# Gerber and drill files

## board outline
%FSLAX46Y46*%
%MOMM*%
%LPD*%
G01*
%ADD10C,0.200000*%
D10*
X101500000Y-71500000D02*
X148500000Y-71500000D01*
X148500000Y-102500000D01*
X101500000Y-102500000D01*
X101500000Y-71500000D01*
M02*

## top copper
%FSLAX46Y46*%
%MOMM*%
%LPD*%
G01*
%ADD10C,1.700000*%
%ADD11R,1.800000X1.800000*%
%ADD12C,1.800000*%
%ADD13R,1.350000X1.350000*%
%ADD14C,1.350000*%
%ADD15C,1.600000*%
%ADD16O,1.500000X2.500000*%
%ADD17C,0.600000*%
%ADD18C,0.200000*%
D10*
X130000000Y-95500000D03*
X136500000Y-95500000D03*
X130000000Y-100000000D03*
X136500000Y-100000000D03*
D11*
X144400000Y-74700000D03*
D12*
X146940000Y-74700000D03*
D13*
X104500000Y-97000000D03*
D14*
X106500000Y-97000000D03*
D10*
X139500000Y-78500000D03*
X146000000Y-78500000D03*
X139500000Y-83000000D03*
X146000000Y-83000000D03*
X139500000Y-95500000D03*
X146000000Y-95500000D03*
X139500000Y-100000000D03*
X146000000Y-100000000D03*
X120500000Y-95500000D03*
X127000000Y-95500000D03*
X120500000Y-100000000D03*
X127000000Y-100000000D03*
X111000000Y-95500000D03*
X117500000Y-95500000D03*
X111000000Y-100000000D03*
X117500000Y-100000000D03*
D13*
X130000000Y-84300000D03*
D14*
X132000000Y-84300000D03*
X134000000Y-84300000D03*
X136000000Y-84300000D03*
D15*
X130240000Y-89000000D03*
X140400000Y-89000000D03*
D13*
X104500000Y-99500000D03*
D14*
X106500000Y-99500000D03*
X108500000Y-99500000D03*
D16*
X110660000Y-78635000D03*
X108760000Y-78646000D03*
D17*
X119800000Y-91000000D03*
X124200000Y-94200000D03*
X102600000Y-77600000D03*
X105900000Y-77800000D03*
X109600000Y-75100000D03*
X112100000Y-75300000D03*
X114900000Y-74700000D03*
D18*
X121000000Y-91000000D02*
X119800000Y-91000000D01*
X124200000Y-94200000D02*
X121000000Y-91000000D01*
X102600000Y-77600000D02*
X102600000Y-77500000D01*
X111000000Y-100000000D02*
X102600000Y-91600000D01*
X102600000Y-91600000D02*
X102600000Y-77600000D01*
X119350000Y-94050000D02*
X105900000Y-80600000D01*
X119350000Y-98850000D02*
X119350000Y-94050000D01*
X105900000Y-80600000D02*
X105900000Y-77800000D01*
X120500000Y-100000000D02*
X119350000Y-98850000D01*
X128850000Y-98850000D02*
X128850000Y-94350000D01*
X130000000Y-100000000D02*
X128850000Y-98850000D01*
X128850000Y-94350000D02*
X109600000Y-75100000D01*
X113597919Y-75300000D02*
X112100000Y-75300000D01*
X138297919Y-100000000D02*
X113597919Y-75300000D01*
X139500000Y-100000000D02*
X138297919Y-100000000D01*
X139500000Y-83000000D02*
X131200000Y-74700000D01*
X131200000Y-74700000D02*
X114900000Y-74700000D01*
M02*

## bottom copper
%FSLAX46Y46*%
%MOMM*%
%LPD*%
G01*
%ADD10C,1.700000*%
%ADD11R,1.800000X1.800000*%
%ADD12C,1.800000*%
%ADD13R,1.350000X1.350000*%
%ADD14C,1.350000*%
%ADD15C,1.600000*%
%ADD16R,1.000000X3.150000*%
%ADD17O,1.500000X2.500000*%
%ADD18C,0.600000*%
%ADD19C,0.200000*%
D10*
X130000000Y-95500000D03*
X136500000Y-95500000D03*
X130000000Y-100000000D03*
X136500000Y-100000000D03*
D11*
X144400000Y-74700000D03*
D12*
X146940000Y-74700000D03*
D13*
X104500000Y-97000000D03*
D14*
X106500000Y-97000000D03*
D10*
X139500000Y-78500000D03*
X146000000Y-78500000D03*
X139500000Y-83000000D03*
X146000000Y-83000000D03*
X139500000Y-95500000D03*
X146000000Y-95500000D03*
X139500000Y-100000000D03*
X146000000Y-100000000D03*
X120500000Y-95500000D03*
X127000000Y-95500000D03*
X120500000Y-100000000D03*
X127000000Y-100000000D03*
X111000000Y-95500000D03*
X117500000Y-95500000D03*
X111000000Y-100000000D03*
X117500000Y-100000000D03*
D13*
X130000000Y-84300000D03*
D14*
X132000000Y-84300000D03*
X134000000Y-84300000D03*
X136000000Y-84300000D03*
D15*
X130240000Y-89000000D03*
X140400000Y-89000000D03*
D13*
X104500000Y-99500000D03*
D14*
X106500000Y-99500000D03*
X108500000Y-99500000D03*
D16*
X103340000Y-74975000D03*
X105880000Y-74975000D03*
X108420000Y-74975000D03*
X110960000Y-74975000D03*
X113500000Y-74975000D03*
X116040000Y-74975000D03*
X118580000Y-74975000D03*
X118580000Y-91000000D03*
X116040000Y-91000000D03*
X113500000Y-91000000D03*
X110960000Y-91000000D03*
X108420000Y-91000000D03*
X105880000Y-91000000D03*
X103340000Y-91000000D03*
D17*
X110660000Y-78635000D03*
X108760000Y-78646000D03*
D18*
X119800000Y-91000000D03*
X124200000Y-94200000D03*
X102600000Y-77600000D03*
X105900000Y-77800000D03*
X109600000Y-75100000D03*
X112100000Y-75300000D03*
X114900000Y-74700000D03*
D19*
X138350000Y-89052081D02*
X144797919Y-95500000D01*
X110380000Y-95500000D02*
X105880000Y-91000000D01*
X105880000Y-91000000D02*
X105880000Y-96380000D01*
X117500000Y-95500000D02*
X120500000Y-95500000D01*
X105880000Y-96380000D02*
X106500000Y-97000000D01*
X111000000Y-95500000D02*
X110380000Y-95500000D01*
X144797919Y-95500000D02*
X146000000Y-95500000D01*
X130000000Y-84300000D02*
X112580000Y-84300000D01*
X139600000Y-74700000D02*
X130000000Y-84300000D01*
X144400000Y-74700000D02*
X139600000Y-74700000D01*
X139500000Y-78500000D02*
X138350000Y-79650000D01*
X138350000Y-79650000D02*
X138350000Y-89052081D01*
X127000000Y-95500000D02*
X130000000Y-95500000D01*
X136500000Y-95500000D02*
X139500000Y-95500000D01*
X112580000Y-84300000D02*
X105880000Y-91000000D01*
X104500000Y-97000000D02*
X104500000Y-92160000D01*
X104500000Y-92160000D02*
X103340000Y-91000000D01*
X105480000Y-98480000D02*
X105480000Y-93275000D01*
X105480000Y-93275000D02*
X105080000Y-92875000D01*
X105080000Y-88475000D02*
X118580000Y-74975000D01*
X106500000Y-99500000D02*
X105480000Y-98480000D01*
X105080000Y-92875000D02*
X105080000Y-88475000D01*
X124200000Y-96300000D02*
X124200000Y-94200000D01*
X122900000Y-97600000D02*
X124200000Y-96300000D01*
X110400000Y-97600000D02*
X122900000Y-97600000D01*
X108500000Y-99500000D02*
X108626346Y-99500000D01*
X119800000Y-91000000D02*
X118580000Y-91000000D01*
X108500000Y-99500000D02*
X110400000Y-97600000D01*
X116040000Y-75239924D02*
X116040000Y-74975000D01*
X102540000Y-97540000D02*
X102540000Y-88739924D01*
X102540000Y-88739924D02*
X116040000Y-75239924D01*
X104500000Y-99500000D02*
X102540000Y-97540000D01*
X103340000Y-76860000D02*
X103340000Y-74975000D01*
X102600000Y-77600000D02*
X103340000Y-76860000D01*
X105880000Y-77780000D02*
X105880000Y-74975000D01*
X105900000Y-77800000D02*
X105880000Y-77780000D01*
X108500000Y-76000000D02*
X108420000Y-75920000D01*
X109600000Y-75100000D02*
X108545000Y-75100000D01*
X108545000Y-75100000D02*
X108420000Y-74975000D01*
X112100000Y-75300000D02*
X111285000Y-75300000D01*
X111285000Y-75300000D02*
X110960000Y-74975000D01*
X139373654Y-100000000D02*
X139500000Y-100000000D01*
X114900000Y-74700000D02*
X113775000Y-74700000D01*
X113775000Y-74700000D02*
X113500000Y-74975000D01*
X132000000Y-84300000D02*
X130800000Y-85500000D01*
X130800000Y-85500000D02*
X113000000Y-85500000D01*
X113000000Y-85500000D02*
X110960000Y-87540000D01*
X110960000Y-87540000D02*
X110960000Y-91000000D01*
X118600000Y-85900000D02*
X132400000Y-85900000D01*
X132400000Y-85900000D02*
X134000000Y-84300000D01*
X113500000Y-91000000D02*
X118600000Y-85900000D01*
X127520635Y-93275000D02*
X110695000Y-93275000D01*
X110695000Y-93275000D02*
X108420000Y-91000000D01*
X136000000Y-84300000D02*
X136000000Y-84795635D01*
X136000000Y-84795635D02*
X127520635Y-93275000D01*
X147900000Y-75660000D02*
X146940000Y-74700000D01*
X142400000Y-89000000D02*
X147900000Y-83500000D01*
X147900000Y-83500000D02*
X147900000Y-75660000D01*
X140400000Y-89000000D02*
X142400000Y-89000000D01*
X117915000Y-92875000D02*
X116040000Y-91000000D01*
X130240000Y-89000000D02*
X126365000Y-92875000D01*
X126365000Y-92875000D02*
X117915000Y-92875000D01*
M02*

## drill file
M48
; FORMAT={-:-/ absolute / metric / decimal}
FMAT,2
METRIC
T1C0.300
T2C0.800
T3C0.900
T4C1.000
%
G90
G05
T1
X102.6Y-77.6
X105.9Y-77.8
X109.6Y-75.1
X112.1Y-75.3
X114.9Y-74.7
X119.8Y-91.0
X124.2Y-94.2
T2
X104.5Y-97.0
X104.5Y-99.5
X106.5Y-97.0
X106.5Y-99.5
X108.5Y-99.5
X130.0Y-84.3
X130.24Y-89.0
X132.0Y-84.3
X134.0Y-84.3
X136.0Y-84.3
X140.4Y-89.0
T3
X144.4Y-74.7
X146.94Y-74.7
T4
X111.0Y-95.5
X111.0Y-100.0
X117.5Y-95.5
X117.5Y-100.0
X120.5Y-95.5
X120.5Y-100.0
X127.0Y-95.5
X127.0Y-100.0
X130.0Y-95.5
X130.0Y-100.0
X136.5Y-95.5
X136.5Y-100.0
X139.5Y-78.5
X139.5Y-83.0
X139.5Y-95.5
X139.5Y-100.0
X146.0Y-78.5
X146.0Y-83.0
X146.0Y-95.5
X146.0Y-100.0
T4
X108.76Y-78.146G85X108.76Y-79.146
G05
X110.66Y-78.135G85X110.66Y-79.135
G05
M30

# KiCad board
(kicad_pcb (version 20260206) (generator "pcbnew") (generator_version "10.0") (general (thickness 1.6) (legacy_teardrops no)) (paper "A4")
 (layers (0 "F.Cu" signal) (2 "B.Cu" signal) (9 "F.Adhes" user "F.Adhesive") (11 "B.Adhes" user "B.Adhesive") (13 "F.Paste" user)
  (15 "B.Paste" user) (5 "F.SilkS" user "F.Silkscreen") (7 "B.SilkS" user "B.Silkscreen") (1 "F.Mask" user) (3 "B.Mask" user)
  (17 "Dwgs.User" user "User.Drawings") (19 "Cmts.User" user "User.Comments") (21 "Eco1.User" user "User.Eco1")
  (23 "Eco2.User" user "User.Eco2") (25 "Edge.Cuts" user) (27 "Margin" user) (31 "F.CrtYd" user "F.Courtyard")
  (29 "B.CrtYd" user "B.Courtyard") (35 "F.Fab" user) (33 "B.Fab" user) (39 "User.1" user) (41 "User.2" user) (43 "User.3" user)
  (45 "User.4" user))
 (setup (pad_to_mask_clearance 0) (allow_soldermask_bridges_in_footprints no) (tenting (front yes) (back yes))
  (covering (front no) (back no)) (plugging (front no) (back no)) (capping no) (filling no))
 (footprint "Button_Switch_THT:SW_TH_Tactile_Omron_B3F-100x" (layer "F.Cu") (at 130 95.5)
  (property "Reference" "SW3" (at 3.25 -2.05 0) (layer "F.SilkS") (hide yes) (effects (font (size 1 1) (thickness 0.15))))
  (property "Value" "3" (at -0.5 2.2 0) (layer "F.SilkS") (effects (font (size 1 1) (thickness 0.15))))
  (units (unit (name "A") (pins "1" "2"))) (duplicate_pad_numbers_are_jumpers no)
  (pad "1" thru_hole circle (at 0 0) (size 1.7 1.7) (drill 1) (layers "*.Cu" "*.Mask") (remove_unused_layers no) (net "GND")
   (thermal_bridge_angle 90))
  (pad "1" thru_hole circle (at 6.5 0) (size 1.7 1.7) (drill 1) (layers "*.Cu" "*.Mask") (remove_unused_layers no) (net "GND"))
  (pad "2" thru_hole circle (at 0 4.5) (size 1.7 1.7) (drill 1) (layers "*.Cu" "*.Mask") (remove_unused_layers no) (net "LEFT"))
  (pad "2" thru_hole circle (at 6.5 4.5) (size 1.7 1.7) (drill 1) (layers "*.Cu" "*.Mask") (remove_unused_layers no) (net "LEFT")))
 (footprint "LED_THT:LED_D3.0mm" (layer "F.Cu") (at 144.4 74.7)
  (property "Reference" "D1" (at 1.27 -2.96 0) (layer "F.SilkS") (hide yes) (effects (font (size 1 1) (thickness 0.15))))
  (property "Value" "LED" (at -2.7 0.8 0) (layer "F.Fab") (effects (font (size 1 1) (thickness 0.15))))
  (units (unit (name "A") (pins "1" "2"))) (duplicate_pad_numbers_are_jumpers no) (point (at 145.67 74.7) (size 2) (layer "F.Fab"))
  (pad "1" thru_hole rect (at 0 0) (size 1.8 1.8) (drill 0.9) (layers "*.Cu" "*.Mask") (remove_unused_layers no) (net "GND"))
  (pad "2" thru_hole circle (at 2.54 0) (size 1.8 1.8) (drill 0.9) (layers "*.Cu" "*.Mask") (remove_unused_layers no) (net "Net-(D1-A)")))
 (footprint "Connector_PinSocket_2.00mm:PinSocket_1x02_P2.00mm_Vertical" (layer "F.Cu") (at 104.5 97 90)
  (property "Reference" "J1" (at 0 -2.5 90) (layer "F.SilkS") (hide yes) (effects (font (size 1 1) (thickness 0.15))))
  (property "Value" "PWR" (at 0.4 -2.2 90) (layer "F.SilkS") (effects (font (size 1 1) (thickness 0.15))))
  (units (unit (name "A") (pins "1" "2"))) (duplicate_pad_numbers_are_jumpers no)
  (pad "1" thru_hole rect (at 0 0 90) (size 1.35 1.35) (drill 0.8) (layers "*.Cu" "*.Mask") (remove_unused_layers no) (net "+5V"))
  (pad "2" thru_hole circle (at 0 2 90) (size 1.35 1.35) (drill 0.8) (layers "*.Cu" "*.Mask") (remove_unused_layers no) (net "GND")))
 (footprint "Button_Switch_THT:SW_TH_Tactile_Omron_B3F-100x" (layer "F.Cu") (at 139.5 78.5)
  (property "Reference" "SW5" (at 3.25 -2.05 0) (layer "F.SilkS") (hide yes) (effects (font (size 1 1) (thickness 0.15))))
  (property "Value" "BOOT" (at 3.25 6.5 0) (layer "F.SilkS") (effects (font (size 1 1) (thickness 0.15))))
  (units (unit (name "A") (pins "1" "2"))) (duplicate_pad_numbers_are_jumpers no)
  (pad "1" thru_hole circle (at 0 0) (size 1.7 1.7) (drill 1) (layers "*.Cu" "*.Mask") (remove_unused_layers no) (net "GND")
   (thermal_bridge_angle 90))
  (pad "1" thru_hole circle (at 6.5 0) (size 1.7 1.7) (drill 1) (layers "*.Cu" "*.Mask") (remove_unused_layers no) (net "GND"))
  (pad "2" thru_hole circle (at 0 4.5) (size 1.7 1.7) (drill 1) (layers "*.Cu" "*.Mask") (remove_unused_layers no) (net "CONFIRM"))
  (pad "2" thru_hole circle (at 6.5 4.5) (size 1.7 1.7) (drill 1) (layers "*.Cu" "*.Mask") (remove_unused_layers no) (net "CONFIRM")))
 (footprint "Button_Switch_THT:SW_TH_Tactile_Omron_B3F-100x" (layer "F.Cu") (at 139.5 95.5)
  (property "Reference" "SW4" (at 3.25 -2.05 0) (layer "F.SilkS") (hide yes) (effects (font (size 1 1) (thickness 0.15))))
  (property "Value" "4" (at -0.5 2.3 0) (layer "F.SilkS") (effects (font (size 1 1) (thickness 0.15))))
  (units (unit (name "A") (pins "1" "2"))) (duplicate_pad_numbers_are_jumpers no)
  (pad "1" thru_hole circle (at 0 0) (size 1.7 1.7) (drill 1) (layers "*.Cu" "*.Mask") (remove_unused_layers no) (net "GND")
   (thermal_bridge_angle 90))
  (pad "1" thru_hole circle (at 6.5 0) (size 1.7 1.7) (drill 1) (layers "*.Cu" "*.Mask") (remove_unused_layers no) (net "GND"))
  (pad "2" thru_hole circle (at 0 4.5) (size 1.7 1.7) (drill 1) (layers "*.Cu" "*.Mask") (remove_unused_layers no) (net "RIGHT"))
  (pad "2" thru_hole circle (at 6.5 4.5) (size 1.7 1.7) (drill 1) (layers "*.Cu" "*.Mask") (remove_unused_layers no) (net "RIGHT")))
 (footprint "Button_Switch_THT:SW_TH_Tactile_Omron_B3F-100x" (layer "F.Cu") (at 120.5 95.5)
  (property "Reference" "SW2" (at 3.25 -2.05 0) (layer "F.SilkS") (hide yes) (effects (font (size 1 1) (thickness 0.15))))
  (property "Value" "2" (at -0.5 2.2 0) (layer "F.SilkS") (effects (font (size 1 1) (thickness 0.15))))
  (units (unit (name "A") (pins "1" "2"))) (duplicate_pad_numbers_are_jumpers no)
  (pad "1" thru_hole circle (at 0 0) (size 1.7 1.7) (drill 1) (layers "*.Cu" "*.Mask") (remove_unused_layers no) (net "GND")
   (thermal_bridge_angle 90))
  (pad "1" thru_hole circle (at 6.5 0) (size 1.7 1.7) (drill 1) (layers "*.Cu" "*.Mask") (remove_unused_layers no) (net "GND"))
  (pad "2" thru_hole circle (at 0 4.5) (size 1.7 1.7) (drill 1) (layers "*.Cu" "*.Mask") (remove_unused_layers no) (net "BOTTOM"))
  (pad "2" thru_hole circle (at 6.5 4.5) (size 1.7 1.7) (drill 1) (layers "*.Cu" "*.Mask") (remove_unused_layers no) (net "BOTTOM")))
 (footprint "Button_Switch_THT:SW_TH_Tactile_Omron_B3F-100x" (layer "F.Cu") (at 111 95.5)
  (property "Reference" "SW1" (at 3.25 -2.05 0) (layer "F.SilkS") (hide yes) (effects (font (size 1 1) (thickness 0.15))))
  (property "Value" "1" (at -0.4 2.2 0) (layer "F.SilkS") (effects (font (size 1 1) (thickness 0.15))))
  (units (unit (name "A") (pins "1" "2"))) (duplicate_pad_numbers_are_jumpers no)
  (pad "1" thru_hole circle (at 0 0) (size 1.7 1.7) (drill 1) (layers "*.Cu" "*.Mask") (remove_unused_layers no) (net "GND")
   (thermal_bridge_angle 90))
  (pad "1" thru_hole circle (at 6.5 0) (size 1.7 1.7) (drill 1) (layers "*.Cu" "*.Mask") (remove_unused_layers no) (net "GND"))
  (pad "2" thru_hole circle (at 0 4.5) (size 1.7 1.7) (drill 1) (layers "*.Cu" "*.Mask") (remove_unused_layers no) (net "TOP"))
  (pad "2" thru_hole circle (at 6.5 4.5) (size 1.7 1.7) (drill 1) (layers "*.Cu" "*.Mask") (remove_unused_layers no) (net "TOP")))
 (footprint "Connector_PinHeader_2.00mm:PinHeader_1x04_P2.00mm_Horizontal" (layer "F.Cu") (at 130 84.3 90)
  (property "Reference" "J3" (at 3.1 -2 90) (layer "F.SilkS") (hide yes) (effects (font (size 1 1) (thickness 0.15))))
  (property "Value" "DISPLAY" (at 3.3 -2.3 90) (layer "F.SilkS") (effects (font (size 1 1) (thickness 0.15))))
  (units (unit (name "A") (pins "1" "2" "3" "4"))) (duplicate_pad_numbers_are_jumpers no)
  (pad "1" thru_hole rect (at 0 0 90) (size 1.35 1.35) (drill 0.8) (layers "*.Cu" "*.Mask") (remove_unused_layers no) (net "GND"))
  (pad "2" thru_hole circle (at 0 2 90) (size 1.35 1.35) (drill 0.8) (layers "*.Cu" "*.Mask") (remove_unused_layers no) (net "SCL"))
  (pad "3" thru_hole circle (at 0 4 90) (size 1.35 1.35) (drill 0.8) (layers "*.Cu" "*.Mask") (remove_unused_layers no) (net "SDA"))
  (pad "4" thru_hole circle (at 0 6 90) (size 1.35 1.35) (drill 0.8) (layers "*.Cu" "*.Mask") (remove_unused_layers no) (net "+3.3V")))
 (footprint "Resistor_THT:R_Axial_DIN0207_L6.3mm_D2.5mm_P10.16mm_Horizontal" (layer "F.Cu") (at 130.24 89)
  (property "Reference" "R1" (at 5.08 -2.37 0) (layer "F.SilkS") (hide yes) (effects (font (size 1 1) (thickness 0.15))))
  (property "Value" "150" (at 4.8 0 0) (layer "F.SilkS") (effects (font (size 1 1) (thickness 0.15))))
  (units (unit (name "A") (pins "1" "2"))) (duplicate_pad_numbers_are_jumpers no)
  (pad "1" thru_hole circle (at 0 0) (size 1.6 1.6) (drill 0.8) (layers "*.Cu" "*.Mask") (remove_unused_layers no) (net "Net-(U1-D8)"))
  (pad "2" thru_hole circle (at 10.16 0) (size 1.6 1.6) (drill 0.8) (layers "*.Cu" "*.Mask") (remove_unused_layers no) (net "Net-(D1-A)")))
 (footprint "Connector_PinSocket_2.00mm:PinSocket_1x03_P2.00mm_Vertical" (layer "F.Cu") (at 104.5 99.5 90)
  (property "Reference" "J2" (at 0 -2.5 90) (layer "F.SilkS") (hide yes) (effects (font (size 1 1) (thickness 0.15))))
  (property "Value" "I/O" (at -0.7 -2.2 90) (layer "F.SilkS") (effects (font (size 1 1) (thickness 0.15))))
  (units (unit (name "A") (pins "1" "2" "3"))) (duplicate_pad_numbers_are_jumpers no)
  (pad "1" thru_hole rect (at 0 0 90) (size 1.35 1.35) (drill 0.8) (layers "*.Cu" "*.Mask") (remove_unused_layers no) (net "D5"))
  (pad "2" thru_hole circle (at 0 2 90) (size 1.35 1.35) (drill 0.8) (layers "*.Cu" "*.Mask") (remove_unused_layers no) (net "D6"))
  (pad "3" thru_hole circle (at 0 4 90) (size 1.35 1.35) (drill 0.8) (layers "*.Cu" "*.Mask") (remove_unused_layers no) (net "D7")))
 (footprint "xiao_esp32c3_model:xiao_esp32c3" (layer "B.Cu") (at 112.76 83.575 -90)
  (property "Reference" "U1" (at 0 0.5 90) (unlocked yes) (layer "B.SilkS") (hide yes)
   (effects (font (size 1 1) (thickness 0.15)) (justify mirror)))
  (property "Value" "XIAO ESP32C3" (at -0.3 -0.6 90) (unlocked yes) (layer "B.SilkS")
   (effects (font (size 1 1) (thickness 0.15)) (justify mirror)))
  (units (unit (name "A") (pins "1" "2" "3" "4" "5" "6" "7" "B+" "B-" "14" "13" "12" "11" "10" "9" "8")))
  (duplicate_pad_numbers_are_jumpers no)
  (pad "1" smd rect (at -8.6 9.42 270) (size 3.15 1) (layers "B.Cu" "B.Mask" "B.Paste") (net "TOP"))
  (pad "2" smd rect (at -8.6 6.88 270) (size 3.15 1) (layers "B.Cu" "B.Mask" "B.Paste") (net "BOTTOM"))
  (pad "3" smd rect (at -8.6 4.34 270) (size 3.15 1) (layers "B.Cu" "B.Mask" "B.Paste") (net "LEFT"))
  (pad "4" smd rect (at -8.6 1.8 270) (size 3.15 1) (layers "B.Cu" "B.Mask" "B.Paste") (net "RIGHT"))
  (pad "5" smd rect (at -8.6 -0.74 270) (size 3.15 1) (layers "B.Cu" "B.Mask" "B.Paste") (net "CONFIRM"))
  (pad "6" smd rect (at -8.6 -3.28 270) (size 3.15 1) (layers "B.Cu" "B.Mask" "B.Paste") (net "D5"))
  (pad "7" smd rect (at -8.6 -5.82 270) (size 3.15 1) (layers "B.Cu" "B.Mask" "B.Paste") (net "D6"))
  (pad "8" smd rect (at 7.425 -5.82 270) (size 3.15 1) (layers "B.Cu" "B.Mask" "B.Paste") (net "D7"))
  (pad "9" smd rect (at 7.425 -3.28 270) (size 3.15 1) (layers "B.Cu" "B.Mask" "B.Paste") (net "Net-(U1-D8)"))
  (pad "10" smd rect (at 7.425 -0.74 270) (size 3.15 1) (layers "B.Cu" "B.Mask" "B.Paste") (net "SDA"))
  (pad "11" smd rect (at 7.425 1.8 270) (size 3.15 1) (layers "B.Cu" "B.Mask" "B.Paste") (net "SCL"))
  (pad "12" smd rect (at 7.425 4.34 270) (size 3.15 1) (layers "B.Cu" "B.Mask" "B.Paste") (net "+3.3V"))
  (pad "13" smd rect (at 7.425 6.88 270) (size 3.15 1) (layers "B.Cu" "B.Mask" "B.Paste") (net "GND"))
  (pad "14" smd rect (at 7.425 9.42 270) (size 3.15 1) (layers "B.Cu" "B.Mask" "B.Paste") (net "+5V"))
  (pad "B+" thru_hole oval (at -4.94 2.1 270) (size 2.5 1.5) (drill oval 2 1) (layers "*.Cu" "*.Mask") (remove_unused_layers no)
   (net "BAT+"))
  (pad "B-" thru_hole oval (at -4.929 4 270) (size 2.5 1.5) (drill oval 2 1) (layers "*.Cu" "*.Mask") (remove_unused_layers no) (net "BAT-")))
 (gr_rect (start 101.5 71.5) (end 148.5 102.5) (stroke (width 0.2) (type default)) (fill no) (layer "Edge.Cuts"))
 (segment (start 138.35 89.052081) (end 144.797919 95.5) (width 0.2) (layer "B.Cu") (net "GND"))
 (segment (start 110.38 95.5) (end 105.88 91) (width 0.2) (layer "B.Cu") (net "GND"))
 (segment (start 105.88 91) (end 105.88 96.38) (width 0.2) (layer "B.Cu") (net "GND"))
 (segment (start 117.5 95.5) (end 120.5 95.5) (width 0.2) (layer "B.Cu") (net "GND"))
 (segment (start 105.88 96.38) (end 106.5 97) (width 0.2) (layer "B.Cu") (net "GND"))
 (segment (start 111 95.5) (end 110.38 95.5) (width 0.2) (layer "B.Cu") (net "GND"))
 (segment (start 144.797919 95.5) (end 146 95.5) (width 0.2) (layer "B.Cu") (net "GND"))
 (segment (start 130 84.3) (end 112.58 84.3) (width 0.2) (layer "B.Cu") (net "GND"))
 (segment (start 139.6 74.7) (end 130 84.3) (width 0.2) (layer "B.Cu") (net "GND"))
 (segment (start 144.4 74.7) (end 139.6 74.7) (width 0.2) (layer "B.Cu") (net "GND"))
 (segment (start 139.5 78.5) (end 138.35 79.65) (width 0.2) (layer "B.Cu") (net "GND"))
 (segment (start 138.35 79.65) (end 138.35 89.052081) (width 0.2) (layer "B.Cu") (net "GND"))
 (segment (start 127 95.5) (end 130 95.5) (width 0.2) (layer "B.Cu") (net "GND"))
 (segment (start 136.5 95.5) (end 139.5 95.5) (width 0.2) (layer "B.Cu") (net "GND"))
 (segment (start 112.58 84.3) (end 105.88 91) (width 0.2) (layer "B.Cu") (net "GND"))
 (segment (start 104.5 97) (end 104.5 92.16) (width 0.2) (layer "B.Cu") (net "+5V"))
 (segment (start 104.5 92.16) (end 103.34 91) (width 0.2) (layer "B.Cu") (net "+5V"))
 (segment (start 105.48 98.48) (end 105.48 93.275) (width 0.2) (layer "B.Cu") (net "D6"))
 (segment (start 105.48 93.275) (end 105.08 92.875) (width 0.2) (layer "B.Cu") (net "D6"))
 (segment (start 105.08 88.475) (end 118.58 74.975) (width 0.2) (layer "B.Cu") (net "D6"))
 (segment (start 106.5 99.5) (end 105.48 98.48) (width 0.2) (layer "B.Cu") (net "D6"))
 (segment (start 105.08 92.875) (end 105.08 88.475) (width 0.2) (layer "B.Cu") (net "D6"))
 (segment (start 121 91) (end 119.8 91) (width 0.2) (layer "F.Cu") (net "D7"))
 (segment (start 124.2 94.2) (end 121 91) (width 0.2) (layer "F.Cu") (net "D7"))
 (via (at 119.8 91) (size 0.6) (drill 0.3) (layers "F.Cu" "B.Cu") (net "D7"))
 (via (at 124.2 94.2) (size 0.6) (drill 0.3) (layers "F.Cu" "B.Cu") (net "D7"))
 (segment (start 124.2 96.3) (end 124.2 94.2) (width 0.2) (layer "B.Cu") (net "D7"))
 (segment (start 122.9 97.6) (end 124.2 96.3) (width 0.2) (layer "B.Cu") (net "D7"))
 (segment (start 110.4 97.6) (end 122.9 97.6) (width 0.2) (layer "B.Cu") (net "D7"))
 (segment (start 108.5 99.5) (end 108.626346 99.5) (width 0.2) (layer "B.Cu") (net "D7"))
 (segment (start 119.8 91) (end 118.58 91) (width 0.2) (layer "B.Cu") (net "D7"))
 (segment (start 108.5 99.5) (end 110.4 97.6) (width 0.2) (layer "B.Cu") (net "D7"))
 (segment (start 116.04 75.239924) (end 116.04 74.975) (width 0.2) (layer "B.Cu") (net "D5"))
 (segment (start 102.54 97.54) (end 102.54 88.739924) (width 0.2) (layer "B.Cu") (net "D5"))
 (segment (start 102.54 88.739924) (end 116.04 75.239924) (width 0.2) (layer "B.Cu") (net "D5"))
 (segment (start 104.5 99.5) (end 102.54 97.54) (width 0.2) (layer "B.Cu") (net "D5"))
 (segment (start 102.6 77.6) (end 102.6 77.5) (width 0.2) (layer "F.Cu") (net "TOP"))
 (segment (start 111 100) (end 102.6 91.6) (width 0.2) (layer "F.Cu") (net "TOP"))
 (segment (start 102.6 91.6) (end 102.6 77.6) (width 0.2) (layer "F.Cu") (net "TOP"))
 (via (at 102.6 77.6) (size 0.6) (drill 0.3) (layers "F.Cu" "B.Cu") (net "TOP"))
 (segment (start 103.34 76.86) (end 103.34 74.975) (width 0.2) (layer "B.Cu") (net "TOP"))
 (segment (start 102.6 77.6) (end 103.34 76.86) (width 0.2) (layer "B.Cu") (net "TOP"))
 (segment (start 119.35 94.05) (end 105.9 80.6) (width 0.2) (layer "F.Cu") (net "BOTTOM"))
 (segment (start 119.35 98.85) (end 119.35 94.05) (width 0.2) (layer "F.Cu") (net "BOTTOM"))
 (segment (start 105.9 80.6) (end 105.9 77.8) (width 0.2) (layer "F.Cu") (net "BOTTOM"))
 (segment (start 120.5 100) (end 119.35 98.85) (width 0.2) (layer "F.Cu") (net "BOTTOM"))
 (via (at 105.9 77.8) (size 0.6) (drill 0.3) (layers "F.Cu" "B.Cu") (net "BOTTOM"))
 (segment (start 105.88 77.78) (end 105.88 74.975) (width 0.2) (layer "B.Cu") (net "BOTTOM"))
 (segment (start 105.9 77.8) (end 105.88 77.78) (width 0.2) (layer "B.Cu") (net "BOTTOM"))
 (segment (start 128.85 98.85) (end 128.85 94.35) (width 0.2) (layer "F.Cu") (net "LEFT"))
 (segment (start 130 100) (end 128.85 98.85) (width 0.2) (layer "F.Cu") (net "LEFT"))
 (segment (start 128.85 94.35) (end 109.6 75.1) (width 0.2) (layer "F.Cu") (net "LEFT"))
 (via (at 109.6 75.1) (size 0.6) (drill 0.3) (layers "F.Cu" "B.Cu") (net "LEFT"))
 (segment (start 108.5 76) (end 108.42 75.92) (width 0.2) (layer "B.Cu") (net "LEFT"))
 (segment (start 109.6 75.1) (end 108.545 75.1) (width 0.2) (layer "B.Cu") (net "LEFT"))
 (segment (start 108.545 75.1) (end 108.42 74.975) (width 0.2) (layer "B.Cu") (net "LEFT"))
 (segment (start 113.597919 75.3) (end 112.1 75.3) (width 0.2) (layer "F.Cu") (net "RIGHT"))
 (segment (start 138.297919 100) (end 113.597919 75.3) (width 0.2) (layer "F.Cu") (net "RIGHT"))
 (segment (start 139.5 100) (end 138.297919 100) (width 0.2) (layer "F.Cu") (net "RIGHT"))
 (via (at 112.1 75.3) (size 0.6) (drill 0.3) (layers "F.Cu" "B.Cu") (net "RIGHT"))
 (segment (start 112.1 75.3) (end 111.285 75.3) (width 0.2) (layer "B.Cu") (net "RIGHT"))
 (segment (start 111.285 75.3) (end 110.96 74.975) (width 0.2) (layer "B.Cu") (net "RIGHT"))
 (segment (start 139.373654 100) (end 139.5 100) (width 0.2) (layer "B.Cu") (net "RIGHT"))
 (segment (start 139.5 83) (end 131.2 74.7) (width 0.2) (layer "F.Cu") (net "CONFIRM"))
 (segment (start 131.2 74.7) (end 114.9 74.7) (width 0.2) (layer "F.Cu") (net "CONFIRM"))
 (via (at 114.9 74.7) (size 0.6) (drill 0.3) (layers "F.Cu" "B.Cu") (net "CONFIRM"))
 (segment (start 114.9 74.7) (end 113.775 74.7) (width 0.2) (layer "B.Cu") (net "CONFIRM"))
 (segment (start 113.775 74.7) (end 113.5 74.975) (width 0.2) (layer "B.Cu") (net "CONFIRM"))
 (segment (start 132 84.3) (end 130.8 85.5) (width 0.2) (layer "B.Cu") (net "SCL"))
 (segment (start 130.8 85.5) (end 113 85.5) (width 0.2) (layer "B.Cu") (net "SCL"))
 (segment (start 113 85.5) (end 110.96 87.54) (width 0.2) (layer "B.Cu") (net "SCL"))
 (segment (start 110.96 87.54) (end 110.96 91) (width 0.2) (layer "B.Cu") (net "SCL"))
 (segment (start 118.6 85.9) (end 132.4 85.9) (width 0.2) (layer "B.Cu") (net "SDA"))
 (segment (start 132.4 85.9) (end 134 84.3) (width 0.2) (layer "B.Cu") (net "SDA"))
 (segment (start 113.5 91) (end 118.6 85.9) (width 0.2) (layer "B.Cu") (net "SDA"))
 (segment (start 127.520635 93.275) (end 110.695 93.275) (width 0.2) (layer "B.Cu") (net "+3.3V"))
 (segment (start 110.695 93.275) (end 108.42 91) (width 0.2) (layer "B.Cu") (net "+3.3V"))
 (segment (start 136 84.3) (end 136 84.795635) (width 0.2) (layer "B.Cu") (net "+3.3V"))
 (segment (start 136 84.795635) (end 127.520635 93.275) (width 0.2) (layer "B.Cu") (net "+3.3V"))
 (segment (start 147.9 75.66) (end 146.94 74.7) (width 0.2) (layer "B.Cu") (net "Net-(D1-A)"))
 (segment (start 142.4 89) (end 147.9 83.5) (width 0.2) (layer "B.Cu") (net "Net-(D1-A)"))
 (segment (start 147.9 83.5) (end 147.9 75.66) (width 0.2) (layer "B.Cu") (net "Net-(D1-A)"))
 (segment (start 140.4 89) (end 142.4 89) (width 0.2) (layer "B.Cu") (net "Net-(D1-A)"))
 (segment (start 117.915 92.875) (end 116.04 91) (width 0.2) (layer "B.Cu") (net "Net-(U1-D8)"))
 (segment (start 130.24 89) (end 126.365 92.875) (width 0.2) (layer "B.Cu") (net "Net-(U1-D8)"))
 (segment (start 126.365 92.875) (end 117.915 92.875) (width 0.2) (layer "B.Cu") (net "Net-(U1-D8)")))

